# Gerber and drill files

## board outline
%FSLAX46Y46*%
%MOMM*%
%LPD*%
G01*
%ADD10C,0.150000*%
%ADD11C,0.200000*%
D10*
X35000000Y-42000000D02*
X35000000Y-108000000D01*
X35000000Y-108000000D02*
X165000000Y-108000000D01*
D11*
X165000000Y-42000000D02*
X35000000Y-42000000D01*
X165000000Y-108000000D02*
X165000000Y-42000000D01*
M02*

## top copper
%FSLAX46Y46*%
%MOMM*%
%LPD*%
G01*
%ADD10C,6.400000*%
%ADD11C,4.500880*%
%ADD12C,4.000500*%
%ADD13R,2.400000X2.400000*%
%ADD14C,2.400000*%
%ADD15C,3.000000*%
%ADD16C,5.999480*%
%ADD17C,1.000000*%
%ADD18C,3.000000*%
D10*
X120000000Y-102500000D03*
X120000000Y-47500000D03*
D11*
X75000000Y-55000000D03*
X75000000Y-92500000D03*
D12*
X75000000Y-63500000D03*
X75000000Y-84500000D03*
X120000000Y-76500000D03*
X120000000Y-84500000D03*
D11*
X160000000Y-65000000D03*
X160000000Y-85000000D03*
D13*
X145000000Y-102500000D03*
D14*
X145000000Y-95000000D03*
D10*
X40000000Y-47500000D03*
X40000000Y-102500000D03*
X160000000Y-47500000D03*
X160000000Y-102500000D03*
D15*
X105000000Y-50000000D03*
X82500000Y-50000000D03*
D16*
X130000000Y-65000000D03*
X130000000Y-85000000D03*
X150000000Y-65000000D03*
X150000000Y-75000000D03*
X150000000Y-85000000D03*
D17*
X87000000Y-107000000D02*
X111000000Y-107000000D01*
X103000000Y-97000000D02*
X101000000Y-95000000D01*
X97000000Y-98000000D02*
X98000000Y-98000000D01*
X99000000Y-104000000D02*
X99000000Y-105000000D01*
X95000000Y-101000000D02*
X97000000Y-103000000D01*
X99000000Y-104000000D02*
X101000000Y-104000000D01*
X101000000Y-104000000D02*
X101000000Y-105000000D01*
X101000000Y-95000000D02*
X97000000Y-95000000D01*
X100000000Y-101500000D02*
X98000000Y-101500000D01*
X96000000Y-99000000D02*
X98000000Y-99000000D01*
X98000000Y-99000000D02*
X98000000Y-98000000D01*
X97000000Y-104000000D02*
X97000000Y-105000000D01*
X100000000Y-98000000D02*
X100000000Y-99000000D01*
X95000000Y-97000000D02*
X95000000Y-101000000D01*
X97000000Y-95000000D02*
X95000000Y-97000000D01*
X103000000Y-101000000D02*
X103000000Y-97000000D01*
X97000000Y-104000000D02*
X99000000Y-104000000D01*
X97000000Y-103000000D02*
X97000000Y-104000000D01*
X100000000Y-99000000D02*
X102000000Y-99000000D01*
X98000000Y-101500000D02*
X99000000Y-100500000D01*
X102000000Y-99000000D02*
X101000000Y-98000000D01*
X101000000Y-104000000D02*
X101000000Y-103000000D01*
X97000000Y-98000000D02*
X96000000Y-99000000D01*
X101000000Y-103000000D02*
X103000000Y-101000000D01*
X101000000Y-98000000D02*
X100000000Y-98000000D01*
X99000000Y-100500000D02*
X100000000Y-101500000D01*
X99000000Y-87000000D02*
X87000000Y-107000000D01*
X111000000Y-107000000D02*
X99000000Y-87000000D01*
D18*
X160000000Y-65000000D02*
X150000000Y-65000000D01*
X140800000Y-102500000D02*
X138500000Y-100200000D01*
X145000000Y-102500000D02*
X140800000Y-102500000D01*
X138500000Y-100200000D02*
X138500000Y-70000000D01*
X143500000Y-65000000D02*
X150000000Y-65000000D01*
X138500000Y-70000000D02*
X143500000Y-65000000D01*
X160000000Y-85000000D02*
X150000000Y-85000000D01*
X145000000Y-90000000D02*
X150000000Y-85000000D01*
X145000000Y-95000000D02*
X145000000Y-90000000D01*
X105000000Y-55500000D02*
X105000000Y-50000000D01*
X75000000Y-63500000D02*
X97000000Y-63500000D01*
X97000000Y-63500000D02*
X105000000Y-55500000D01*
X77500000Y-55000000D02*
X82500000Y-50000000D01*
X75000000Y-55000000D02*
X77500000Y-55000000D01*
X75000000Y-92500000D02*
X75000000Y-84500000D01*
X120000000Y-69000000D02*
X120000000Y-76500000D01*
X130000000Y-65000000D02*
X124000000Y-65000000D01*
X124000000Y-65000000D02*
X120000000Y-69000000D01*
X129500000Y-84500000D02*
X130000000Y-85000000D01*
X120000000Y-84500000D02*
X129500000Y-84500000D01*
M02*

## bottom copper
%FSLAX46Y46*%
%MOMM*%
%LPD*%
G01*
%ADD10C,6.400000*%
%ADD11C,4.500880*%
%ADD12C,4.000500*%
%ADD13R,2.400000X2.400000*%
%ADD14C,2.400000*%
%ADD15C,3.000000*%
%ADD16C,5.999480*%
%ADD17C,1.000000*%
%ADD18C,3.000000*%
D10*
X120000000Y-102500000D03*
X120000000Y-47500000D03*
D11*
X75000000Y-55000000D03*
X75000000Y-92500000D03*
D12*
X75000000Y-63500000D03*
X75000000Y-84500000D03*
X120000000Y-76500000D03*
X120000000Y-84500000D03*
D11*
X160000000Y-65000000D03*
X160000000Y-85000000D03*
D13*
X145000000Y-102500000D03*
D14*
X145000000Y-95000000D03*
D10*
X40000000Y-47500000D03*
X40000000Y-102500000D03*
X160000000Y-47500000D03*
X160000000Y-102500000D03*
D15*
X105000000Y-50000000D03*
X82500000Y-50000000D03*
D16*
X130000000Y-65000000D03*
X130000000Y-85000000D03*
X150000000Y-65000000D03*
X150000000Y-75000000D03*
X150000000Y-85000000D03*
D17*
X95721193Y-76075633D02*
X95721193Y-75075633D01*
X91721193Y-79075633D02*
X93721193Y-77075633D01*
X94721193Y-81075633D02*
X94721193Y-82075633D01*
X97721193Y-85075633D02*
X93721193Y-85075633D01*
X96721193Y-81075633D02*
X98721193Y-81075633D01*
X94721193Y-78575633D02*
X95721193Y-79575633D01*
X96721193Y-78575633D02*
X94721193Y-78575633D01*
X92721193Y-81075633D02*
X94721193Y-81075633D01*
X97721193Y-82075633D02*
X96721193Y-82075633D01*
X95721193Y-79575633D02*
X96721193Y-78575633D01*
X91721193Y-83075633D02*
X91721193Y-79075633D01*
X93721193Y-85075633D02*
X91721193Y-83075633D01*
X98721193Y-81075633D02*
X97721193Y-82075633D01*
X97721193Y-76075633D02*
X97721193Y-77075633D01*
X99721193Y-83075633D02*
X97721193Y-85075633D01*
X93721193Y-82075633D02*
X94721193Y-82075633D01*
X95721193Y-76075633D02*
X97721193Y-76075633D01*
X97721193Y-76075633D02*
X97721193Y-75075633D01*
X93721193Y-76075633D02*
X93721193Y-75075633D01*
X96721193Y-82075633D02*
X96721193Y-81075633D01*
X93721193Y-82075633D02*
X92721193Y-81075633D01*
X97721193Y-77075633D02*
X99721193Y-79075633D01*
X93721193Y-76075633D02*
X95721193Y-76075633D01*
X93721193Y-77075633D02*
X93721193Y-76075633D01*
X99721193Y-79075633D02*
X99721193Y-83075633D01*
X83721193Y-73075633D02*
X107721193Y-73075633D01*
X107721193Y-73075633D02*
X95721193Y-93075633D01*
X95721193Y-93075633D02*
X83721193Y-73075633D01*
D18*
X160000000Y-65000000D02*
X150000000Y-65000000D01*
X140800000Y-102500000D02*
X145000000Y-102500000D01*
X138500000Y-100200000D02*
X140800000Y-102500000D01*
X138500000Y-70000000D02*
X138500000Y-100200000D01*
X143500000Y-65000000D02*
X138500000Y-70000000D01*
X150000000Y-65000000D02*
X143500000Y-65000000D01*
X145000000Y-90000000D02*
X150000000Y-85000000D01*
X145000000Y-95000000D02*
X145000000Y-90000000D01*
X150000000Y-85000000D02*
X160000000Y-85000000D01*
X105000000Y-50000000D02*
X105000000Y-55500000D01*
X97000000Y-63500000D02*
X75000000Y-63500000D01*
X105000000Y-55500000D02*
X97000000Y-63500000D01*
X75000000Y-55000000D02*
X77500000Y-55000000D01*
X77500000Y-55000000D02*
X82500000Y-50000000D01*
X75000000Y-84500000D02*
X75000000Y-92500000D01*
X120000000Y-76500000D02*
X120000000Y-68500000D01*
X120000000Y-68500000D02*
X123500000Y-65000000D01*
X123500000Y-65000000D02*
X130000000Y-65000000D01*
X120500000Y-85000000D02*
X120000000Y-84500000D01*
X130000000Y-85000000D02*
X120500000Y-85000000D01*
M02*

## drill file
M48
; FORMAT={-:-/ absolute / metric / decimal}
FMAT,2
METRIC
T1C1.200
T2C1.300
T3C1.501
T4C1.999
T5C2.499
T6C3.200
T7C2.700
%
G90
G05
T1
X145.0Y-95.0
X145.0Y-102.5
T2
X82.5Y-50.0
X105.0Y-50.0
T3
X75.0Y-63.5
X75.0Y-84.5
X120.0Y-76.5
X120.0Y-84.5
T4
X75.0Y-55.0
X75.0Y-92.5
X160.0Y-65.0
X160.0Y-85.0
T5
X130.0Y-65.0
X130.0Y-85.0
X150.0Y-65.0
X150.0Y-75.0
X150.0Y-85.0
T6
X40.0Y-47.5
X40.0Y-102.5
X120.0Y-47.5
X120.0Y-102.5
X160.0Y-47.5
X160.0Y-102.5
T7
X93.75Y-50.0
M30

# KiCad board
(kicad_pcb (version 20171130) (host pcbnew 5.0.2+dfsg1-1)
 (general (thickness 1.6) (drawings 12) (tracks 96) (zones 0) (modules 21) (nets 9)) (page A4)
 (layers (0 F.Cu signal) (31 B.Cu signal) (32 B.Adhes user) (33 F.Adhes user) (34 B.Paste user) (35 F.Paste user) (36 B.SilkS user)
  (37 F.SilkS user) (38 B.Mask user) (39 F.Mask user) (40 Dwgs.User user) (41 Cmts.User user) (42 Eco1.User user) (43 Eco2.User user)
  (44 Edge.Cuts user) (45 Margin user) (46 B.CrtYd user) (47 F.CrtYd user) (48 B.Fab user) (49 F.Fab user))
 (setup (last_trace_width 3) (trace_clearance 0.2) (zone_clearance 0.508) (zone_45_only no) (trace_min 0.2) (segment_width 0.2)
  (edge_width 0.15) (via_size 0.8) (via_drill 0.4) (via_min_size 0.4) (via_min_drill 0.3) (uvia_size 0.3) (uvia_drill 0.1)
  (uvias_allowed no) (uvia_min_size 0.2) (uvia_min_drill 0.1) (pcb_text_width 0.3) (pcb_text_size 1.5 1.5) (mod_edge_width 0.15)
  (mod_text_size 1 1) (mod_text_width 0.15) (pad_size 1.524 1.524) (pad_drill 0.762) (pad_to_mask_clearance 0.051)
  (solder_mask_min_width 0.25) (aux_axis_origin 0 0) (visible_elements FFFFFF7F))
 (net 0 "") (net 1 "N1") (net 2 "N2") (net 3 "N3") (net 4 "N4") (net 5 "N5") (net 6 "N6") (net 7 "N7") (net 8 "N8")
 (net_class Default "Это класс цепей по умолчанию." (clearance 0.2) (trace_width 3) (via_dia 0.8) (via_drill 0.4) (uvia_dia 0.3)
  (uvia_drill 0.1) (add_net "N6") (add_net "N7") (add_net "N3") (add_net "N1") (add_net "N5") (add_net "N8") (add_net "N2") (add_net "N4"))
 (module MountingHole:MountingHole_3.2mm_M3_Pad (layer F.Cu) (at 120 102.5)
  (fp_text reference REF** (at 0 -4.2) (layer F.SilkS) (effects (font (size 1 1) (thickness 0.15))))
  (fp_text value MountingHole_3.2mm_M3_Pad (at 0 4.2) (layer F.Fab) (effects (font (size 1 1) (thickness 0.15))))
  (pad 1 thru_hole circle (at 0 0) (size 6.4 6.4) (drill 3.2) (layers *.Cu *.Mask)))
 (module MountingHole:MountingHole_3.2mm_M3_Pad (layer F.Cu) (at 120 47.5)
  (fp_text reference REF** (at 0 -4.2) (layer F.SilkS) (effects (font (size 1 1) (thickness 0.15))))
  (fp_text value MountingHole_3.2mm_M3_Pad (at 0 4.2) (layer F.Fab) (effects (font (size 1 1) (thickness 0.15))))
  (pad 1 thru_hole circle (at 0 0) (size 6.4 6.4) (drill 3.2) (layers *.Cu *.Mask)))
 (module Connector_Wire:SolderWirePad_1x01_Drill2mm (layer F.Cu) (at 75 55)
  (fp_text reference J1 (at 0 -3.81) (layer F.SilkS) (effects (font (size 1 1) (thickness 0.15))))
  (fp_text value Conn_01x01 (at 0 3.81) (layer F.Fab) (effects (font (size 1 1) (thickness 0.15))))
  (pad 1 thru_hole circle (at 0 0) (size 4.50088 4.50088) (drill 1.99898) (layers *.Cu *.Mask) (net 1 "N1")))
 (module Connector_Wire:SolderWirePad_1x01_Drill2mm (layer F.Cu) (at 75 92.5)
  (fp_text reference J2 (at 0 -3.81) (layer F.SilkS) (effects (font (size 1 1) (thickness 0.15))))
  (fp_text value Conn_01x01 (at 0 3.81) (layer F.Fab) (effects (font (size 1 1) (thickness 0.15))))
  (pad 1 thru_hole circle (at 0 0) (size 4.50088 4.50088) (drill 1.99898) (layers *.Cu *.Mask) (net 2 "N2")))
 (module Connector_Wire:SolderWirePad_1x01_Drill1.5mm (layer F.Cu) (at 75 63.5)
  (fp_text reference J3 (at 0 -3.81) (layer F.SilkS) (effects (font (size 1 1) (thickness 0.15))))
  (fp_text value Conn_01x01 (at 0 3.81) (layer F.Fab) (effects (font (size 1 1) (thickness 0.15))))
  (pad 1 thru_hole circle (at 0 0) (size 4.0005 4.0005) (drill 1.50114) (layers *.Cu *.Mask) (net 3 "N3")))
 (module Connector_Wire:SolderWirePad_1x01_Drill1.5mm (layer F.Cu) (at 75 84.5)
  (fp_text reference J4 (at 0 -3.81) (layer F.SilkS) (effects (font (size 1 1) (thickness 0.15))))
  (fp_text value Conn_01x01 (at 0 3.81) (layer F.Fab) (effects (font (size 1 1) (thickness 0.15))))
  (pad 1 thru_hole circle (at 0 0) (size 4.0005 4.0005) (drill 1.50114) (layers *.Cu *.Mask) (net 2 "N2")))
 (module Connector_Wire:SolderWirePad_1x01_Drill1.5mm (layer F.Cu) (at 120 76.5)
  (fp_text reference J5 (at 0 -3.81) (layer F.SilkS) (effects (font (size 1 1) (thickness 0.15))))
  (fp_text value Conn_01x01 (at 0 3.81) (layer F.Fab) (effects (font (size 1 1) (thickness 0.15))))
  (pad 1 thru_hole circle (at 0 0) (size 4.0005 4.0005) (drill 1.50114) (layers *.Cu *.Mask) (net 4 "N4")))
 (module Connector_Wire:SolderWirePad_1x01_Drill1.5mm (layer F.Cu) (at 120 84.5)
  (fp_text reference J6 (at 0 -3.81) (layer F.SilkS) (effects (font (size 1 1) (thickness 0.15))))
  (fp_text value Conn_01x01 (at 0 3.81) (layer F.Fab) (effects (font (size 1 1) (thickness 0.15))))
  (pad 1 thru_hole circle (at 0 0) (size 4.0005 4.0005) (drill 1.50114) (layers *.Cu *.Mask) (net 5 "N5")))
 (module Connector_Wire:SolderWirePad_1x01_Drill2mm (layer F.Cu) (at 160 65)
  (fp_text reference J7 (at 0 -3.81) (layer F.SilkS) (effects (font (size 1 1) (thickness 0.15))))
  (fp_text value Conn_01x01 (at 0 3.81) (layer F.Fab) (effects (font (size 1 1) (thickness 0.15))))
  (pad 1 thru_hole circle (at 0 0) (size 4.50088 4.50088) (drill 1.99898) (layers *.Cu *.Mask) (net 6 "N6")))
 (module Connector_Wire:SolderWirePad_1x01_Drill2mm (layer F.Cu) (at 160 85)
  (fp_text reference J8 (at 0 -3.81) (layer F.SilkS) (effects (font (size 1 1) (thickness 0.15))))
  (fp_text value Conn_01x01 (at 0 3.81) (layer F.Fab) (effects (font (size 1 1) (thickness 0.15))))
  (pad 1 thru_hole circle (at 0 0) (size 4.50088 4.50088) (drill 1.99898) (layers *.Cu *.Mask) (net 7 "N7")))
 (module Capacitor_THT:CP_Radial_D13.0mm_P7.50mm (layer F.Cu) (at 145 102.5 90)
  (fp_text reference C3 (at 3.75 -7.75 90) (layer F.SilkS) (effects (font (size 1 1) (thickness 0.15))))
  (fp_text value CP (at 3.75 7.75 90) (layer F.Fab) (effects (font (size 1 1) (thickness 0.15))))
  (pad 1 thru_hole rect (at 0 0 90) (size 2.4 2.4) (drill 1.2) (layers *.Cu *.Mask) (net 6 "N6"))
  (pad 2 thru_hole circle (at 7.5 0 90) (size 2.4 2.4) (drill 1.2) (layers *.Cu *.Mask) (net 7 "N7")))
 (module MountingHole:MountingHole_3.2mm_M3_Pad (layer F.Cu) (at 40 47.5)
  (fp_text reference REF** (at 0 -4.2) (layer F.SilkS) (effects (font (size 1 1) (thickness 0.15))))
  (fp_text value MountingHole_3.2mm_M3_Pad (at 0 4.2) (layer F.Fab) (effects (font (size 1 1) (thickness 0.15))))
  (pad 1 thru_hole circle (at 0 0) (size 6.4 6.4) (drill 3.2) (layers *.Cu *.Mask)))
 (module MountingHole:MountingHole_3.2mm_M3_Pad (layer F.Cu) (at 40 102.5)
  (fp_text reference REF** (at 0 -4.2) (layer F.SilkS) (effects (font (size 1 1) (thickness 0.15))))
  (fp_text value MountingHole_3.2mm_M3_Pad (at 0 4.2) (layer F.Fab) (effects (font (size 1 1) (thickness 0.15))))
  (pad 1 thru_hole circle (at 0 0) (size 6.4 6.4) (drill 3.2) (layers *.Cu *.Mask)))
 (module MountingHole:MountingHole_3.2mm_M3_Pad (layer F.Cu) (at 160 47.5)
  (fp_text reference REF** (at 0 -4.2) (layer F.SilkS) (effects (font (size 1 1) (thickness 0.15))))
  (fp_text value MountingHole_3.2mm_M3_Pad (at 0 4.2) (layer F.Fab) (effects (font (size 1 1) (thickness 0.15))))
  (pad 1 thru_hole circle (at 0 0) (size 6.4 6.4) (drill 3.2) (layers *.Cu *.Mask)))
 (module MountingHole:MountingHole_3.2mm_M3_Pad (layer F.Cu) (at 160 102.5)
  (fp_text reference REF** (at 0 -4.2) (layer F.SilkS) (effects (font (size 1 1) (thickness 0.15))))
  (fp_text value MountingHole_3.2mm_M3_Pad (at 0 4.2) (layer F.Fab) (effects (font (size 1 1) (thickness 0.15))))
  (pad 1 thru_hole circle (at 0 0) (size 6.4 6.4) (drill 3.2) (layers *.Cu *.Mask)))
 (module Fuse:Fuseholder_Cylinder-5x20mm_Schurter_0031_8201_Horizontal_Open (layer F.Cu) (at 105 50 180)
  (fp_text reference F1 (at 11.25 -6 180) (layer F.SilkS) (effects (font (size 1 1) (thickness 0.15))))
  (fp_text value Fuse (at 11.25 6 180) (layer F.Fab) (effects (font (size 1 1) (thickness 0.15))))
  (pad 1 thru_hole circle (at 0 0 180) (size 3 3) (drill 1.3) (layers *.Cu *.Mask) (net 3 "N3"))
  (pad 2 thru_hole circle (at 22.5 0 180) (size 3 3) (drill 1.3) (layers *.Cu *.Mask) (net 1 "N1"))
  (pad "" np_thru_hole circle (at 11.25 0 180) (size 2.7 2.7) (drill 2.7) (layers *.Cu *.Mask)))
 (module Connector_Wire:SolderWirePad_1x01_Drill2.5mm (layer F.Cu) (at 130 65)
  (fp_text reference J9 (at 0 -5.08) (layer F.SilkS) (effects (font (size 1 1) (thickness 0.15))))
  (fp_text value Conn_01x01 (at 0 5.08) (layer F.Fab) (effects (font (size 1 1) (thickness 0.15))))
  (pad 1 thru_hole circle (at 0 0) (size 5.99948 5.99948) (drill 2.49936) (layers *.Cu *.Mask) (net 4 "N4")))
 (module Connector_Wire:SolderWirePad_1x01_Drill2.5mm (layer F.Cu) (at 130 85)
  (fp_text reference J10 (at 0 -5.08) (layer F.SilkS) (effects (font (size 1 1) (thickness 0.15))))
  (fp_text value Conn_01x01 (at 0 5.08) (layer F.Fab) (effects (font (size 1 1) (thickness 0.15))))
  (pad 1 thru_hole circle (at 0 0) (size 5.99948 5.99948) (drill 2.49936) (layers *.Cu *.Mask) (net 5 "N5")))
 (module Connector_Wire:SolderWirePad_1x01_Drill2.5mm (layer F.Cu) (at 150 65)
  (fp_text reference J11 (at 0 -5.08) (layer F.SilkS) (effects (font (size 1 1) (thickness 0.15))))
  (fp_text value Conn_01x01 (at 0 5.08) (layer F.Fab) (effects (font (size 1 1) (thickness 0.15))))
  (pad 1 thru_hole circle (at 0 0) (size 5.99948 5.99948) (drill 2.49936) (layers *.Cu *.Mask) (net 6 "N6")))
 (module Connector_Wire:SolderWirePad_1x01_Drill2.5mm (layer F.Cu) (at 150 75)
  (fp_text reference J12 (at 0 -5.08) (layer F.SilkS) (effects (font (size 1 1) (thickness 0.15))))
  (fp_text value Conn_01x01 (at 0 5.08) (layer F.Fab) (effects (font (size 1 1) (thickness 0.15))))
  (pad 1 thru_hole circle (at 0 0) (size 5.99948 5.99948) (drill 2.49936) (layers *.Cu *.Mask) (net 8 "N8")))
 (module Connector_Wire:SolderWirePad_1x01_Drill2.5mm (layer F.Cu) (at 150 85)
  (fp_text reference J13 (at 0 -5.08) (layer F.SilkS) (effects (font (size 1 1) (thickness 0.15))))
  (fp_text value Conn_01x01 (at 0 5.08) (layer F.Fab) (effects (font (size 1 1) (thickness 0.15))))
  (pad 1 thru_hole circle (at 0 0) (size 5.99948 5.99948) (drill 2.49936) (layers *.Cu *.Mask) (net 7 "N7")))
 (gr_line (start 35 42) (end 35 108) (layer Edge.Cuts) (width 0.15))
 (gr_line (start 35 108) (end 165 108) (layer Edge.Cuts) (width 0.15))
 (gr_line (start 165 42) (end 35 42) (layer Edge.Cuts) (width 0.2))
 (gr_line (start 165 108) (end 165 42) (layer Edge.Cuts) (width 0.2))
 (segment (start 95.721193 76.075633) (end 95.721193 75.075633) (width 1) (layer B.Cu) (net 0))
 (segment (start 91.721193 79.075633) (end 93.721193 77.075633) (width 1) (layer B.Cu) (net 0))
 (segment (start 94.721193 81.075633) (end 94.721193 82.075633) (width 1) (layer B.Cu) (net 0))
 (segment (start 97.721193 85.075633) (end 93.721193 85.075633) (width 1) (layer B.Cu) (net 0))
 (segment (start 96.721193 81.075633) (end 98.721193 81.075633) (width 1) (layer B.Cu) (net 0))
 (segment (start 94.721193 78.575633) (end 95.721193 79.575633) (width 1) (layer B.Cu) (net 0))
 (segment (start 96.721193 78.575633) (end 94.721193 78.575633) (width 1) (layer B.Cu) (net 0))
 (segment (start 92.721193 81.075633) (end 94.721193 81.075633) (width 1) (layer B.Cu) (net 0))
 (segment (start 97.721193 82.075633) (end 96.721193 82.075633) (width 1) (layer B.Cu) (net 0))
 (segment (start 95.721193 79.575633) (end 96.721193 78.575633) (width 1) (layer B.Cu) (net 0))
 (segment (start 91.721193 83.075633) (end 91.721193 79.075633) (width 1) (layer B.Cu) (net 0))
 (segment (start 93.721193 85.075633) (end 91.721193 83.075633) (width 1) (layer B.Cu) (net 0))
 (segment (start 98.721193 81.075633) (end 97.721193 82.075633) (width 1) (layer B.Cu) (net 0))
 (segment (start 97.721193 76.075633) (end 97.721193 77.075633) (width 1) (layer B.Cu) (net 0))
 (segment (start 99.721193 83.075633) (end 97.721193 85.075633) (width 1) (layer B.Cu) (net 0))
 (segment (start 93.721193 82.075633) (end 94.721193 82.075633) (width 1) (layer B.Cu) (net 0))
 (segment (start 95.721193 76.075633) (end 97.721193 76.075633) (width 1) (layer B.Cu) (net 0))
 (segment (start 97.721193 76.075633) (end 97.721193 75.075633) (width 1) (layer B.Cu) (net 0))
 (segment (start 93.721193 76.075633) (end 93.721193 75.075633) (width 1) (layer B.Cu) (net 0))
 (segment (start 96.721193 82.075633) (end 96.721193 81.075633) (width 1) (layer B.Cu) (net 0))
 (segment (start 93.721193 82.075633) (end 92.721193 81.075633) (width 1) (layer B.Cu) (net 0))
 (segment (start 97.721193 77.075633) (end 99.721193 79.075633) (width 1) (layer B.Cu) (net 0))
 (segment (start 93.721193 76.075633) (end 95.721193 76.075633) (width 1) (layer B.Cu) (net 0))
 (segment (start 93.721193 77.075633) (end 93.721193 76.075633) (width 1) (layer B.Cu) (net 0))
 (segment (start 99.721193 79.075633) (end 99.721193 83.075633) (width 1) (layer B.Cu) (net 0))
 (segment (start 83.721193 73.075633) (end 107.721193 73.075633) (width 1) (layer B.Cu) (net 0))
 (segment (start 107.721193 73.075633) (end 95.721193 93.075633) (width 1) (layer B.Cu) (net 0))
 (segment (start 95.721193 93.075633) (end 83.721193 73.075633) (width 1) (layer B.Cu) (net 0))
 (segment (start 87 107) (end 111 107) (width 1) (layer F.Cu) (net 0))
 (segment (start 103 97) (end 101 95) (width 1) (layer F.Cu) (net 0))
 (segment (start 97 98) (end 98 98) (width 1) (layer F.Cu) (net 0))
 (segment (start 99 104) (end 99 105) (width 1) (layer F.Cu) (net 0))
 (segment (start 95 101) (end 97 103) (width 1) (layer F.Cu) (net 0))
 (segment (start 99 104) (end 101 104) (width 1) (layer F.Cu) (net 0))
 (segment (start 101 104) (end 101 105) (width 1) (layer F.Cu) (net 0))
 (segment (start 101 95) (end 97 95) (width 1) (layer F.Cu) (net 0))
 (segment (start 100 101.5) (end 98 101.5) (width 1) (layer F.Cu) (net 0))
 (segment (start 96 99) (end 98 99) (width 1) (layer F.Cu) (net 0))
 (segment (start 98 99) (end 98 98) (width 1) (layer F.Cu) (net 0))
 (segment (start 97 104) (end 97 105) (width 1) (layer F.Cu) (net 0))
 (segment (start 100 98) (end 100 99) (width 1) (layer F.Cu) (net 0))
 (segment (start 95 97) (end 95 101) (width 1) (layer F.Cu) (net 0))
 (segment (start 97 95) (end 95 97) (width 1) (layer F.Cu) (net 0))
 (segment (start 103 101) (end 103 97) (width 1) (layer F.Cu) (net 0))
 (segment (start 97 104) (end 99 104) (width 1) (layer F.Cu) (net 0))
 (segment (start 97 103) (end 97 104) (width 1) (layer F.Cu) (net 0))
 (segment (start 100 99) (end 102 99) (width 1) (layer F.Cu) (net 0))
 (segment (start 98 101.5) (end 99 100.5) (width 1) (layer F.Cu) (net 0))
 (segment (start 102 99) (end 101 98) (width 1) (layer F.Cu) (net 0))
 (segment (start 101 104) (end 101 103) (width 1) (layer F.Cu) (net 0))
 (segment (start 97 98) (end 96 99) (width 1) (layer F.Cu) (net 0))
 (segment (start 101 103) (end 103 101) (width 1) (layer F.Cu) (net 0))
 (segment (start 101 98) (end 100 98) (width 1) (layer F.Cu) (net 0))
 (segment (start 99 100.5) (end 100 101.5) (width 1) (layer F.Cu) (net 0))
 (segment (start 99 87) (end 87 107) (width 1) (layer F.Cu) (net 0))
 (segment (start 111 107) (end 99 87) (width 1) (layer F.Cu) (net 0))
 (segment (start 160 65) (end 150 65) (width 3) (layer F.Cu) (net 6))
 (segment (start 140.8 102.5) (end 138.5 100.2) (width 3) (layer F.Cu) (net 6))
 (segment (start 145 102.5) (end 140.8 102.5) (width 3) (layer F.Cu) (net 6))
 (segment (start 138.5 100.2) (end 138.5 70) (width 3) (layer F.Cu) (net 6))
 (segment (start 143.5 65) (end 150 65) (width 3) (layer F.Cu) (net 6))
 (segment (start 138.5 70) (end 143.5 65) (width 3) (layer F.Cu) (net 6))
 (segment (start 160 65) (end 150 65) (width 3) (layer B.Cu) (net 6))
 (segment (start 140.8 102.5) (end 145 102.5) (width 3) (layer B.Cu) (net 6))
 (segment (start 138.5 100.2) (end 140.8 102.5) (width 3) (layer B.Cu) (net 6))
 (segment (start 138.5 70) (end 138.5 100.2) (width 3) (layer B.Cu) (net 6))
 (segment (start 143.5 65) (end 138.5 70) (width 3) (layer B.Cu) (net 6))
 (segment (start 150 65) (end 143.5 65) (width 3) (layer B.Cu) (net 6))
 (segment (start 160 85) (end 150 85) (width 3) (layer F.Cu) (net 7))
 (segment (start 145 90) (end 150 85) (width 3) (layer F.Cu) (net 7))
 (segment (start 145 95) (end 145 90) (width 3) (layer F.Cu) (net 7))
 (segment (start 145 90) (end 150 85) (width 3) (layer B.Cu) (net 7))
 (segment (start 145 95) (end 145 90) (width 3) (layer B.Cu) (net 7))
 (segment (start 150 85) (end 160 85) (width 3) (layer B.Cu) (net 7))
 (segment (start 105 55.5) (end 105 50) (width 3) (layer F.Cu) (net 3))
 (segment (start 75 63.5) (end 97 63.5) (width 3) (layer F.Cu) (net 3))
 (segment (start 97 63.5) (end 105 55.5) (width 3) (layer F.Cu) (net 3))
 (segment (start 105 50) (end 105 55.5) (width 3) (layer B.Cu) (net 3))
 (segment (start 97 63.5) (end 75 63.5) (width 3) (layer B.Cu) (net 3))
 (segment (start 105 55.5) (end 97 63.5) (width 3) (layer B.Cu) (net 3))
 (segment (start 77.5 55) (end 82.5 50) (width 3) (layer F.Cu) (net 1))
 (segment (start 75 55) (end 77.5 55) (width 3) (layer F.Cu) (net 1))
 (segment (start 75 55) (end 77.5 55) (width 3) (layer B.Cu) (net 1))
 (segment (start 77.5 55) (end 82.5 50) (width 3) (layer B.Cu) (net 1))
 (segment (start 75 92.5) (end 75 84.5) (width 3) (layer F.Cu) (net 2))
 (segment (start 75 84.5) (end 75 92.5) (width 3) (layer B.Cu) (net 2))
 (segment (start 120 69) (end 120 76.5) (width 3) (layer F.Cu) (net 4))
 (segment (start 130 65) (end 124 65) (width 3) (layer F.Cu) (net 4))
 (segment (start 124 65) (end 120 69) (width 3) (layer F.Cu) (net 4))
 (segment (start 120 76.5) (end 120 68.5) (width 3) (layer B.Cu) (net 4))
 (segment (start 120 68.5) (end 123.5 65) (width 3) (layer B.Cu) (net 4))
 (segment (start 123.5 65) (end 130 65) (width 3) (layer B.Cu) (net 4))
 (segment (start 129.5 84.5) (end 130 85) (width 3) (layer F.Cu) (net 5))
 (segment (start 120 84.5) (end 129.5 84.5) (width 3) (layer F.Cu) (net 5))
 (segment (start 120.5 85) (end 120 84.5) (width 3) (layer B.Cu) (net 5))
 (segment (start 130 85) (end 120.5 85) (width 3) (layer B.Cu) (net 5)))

